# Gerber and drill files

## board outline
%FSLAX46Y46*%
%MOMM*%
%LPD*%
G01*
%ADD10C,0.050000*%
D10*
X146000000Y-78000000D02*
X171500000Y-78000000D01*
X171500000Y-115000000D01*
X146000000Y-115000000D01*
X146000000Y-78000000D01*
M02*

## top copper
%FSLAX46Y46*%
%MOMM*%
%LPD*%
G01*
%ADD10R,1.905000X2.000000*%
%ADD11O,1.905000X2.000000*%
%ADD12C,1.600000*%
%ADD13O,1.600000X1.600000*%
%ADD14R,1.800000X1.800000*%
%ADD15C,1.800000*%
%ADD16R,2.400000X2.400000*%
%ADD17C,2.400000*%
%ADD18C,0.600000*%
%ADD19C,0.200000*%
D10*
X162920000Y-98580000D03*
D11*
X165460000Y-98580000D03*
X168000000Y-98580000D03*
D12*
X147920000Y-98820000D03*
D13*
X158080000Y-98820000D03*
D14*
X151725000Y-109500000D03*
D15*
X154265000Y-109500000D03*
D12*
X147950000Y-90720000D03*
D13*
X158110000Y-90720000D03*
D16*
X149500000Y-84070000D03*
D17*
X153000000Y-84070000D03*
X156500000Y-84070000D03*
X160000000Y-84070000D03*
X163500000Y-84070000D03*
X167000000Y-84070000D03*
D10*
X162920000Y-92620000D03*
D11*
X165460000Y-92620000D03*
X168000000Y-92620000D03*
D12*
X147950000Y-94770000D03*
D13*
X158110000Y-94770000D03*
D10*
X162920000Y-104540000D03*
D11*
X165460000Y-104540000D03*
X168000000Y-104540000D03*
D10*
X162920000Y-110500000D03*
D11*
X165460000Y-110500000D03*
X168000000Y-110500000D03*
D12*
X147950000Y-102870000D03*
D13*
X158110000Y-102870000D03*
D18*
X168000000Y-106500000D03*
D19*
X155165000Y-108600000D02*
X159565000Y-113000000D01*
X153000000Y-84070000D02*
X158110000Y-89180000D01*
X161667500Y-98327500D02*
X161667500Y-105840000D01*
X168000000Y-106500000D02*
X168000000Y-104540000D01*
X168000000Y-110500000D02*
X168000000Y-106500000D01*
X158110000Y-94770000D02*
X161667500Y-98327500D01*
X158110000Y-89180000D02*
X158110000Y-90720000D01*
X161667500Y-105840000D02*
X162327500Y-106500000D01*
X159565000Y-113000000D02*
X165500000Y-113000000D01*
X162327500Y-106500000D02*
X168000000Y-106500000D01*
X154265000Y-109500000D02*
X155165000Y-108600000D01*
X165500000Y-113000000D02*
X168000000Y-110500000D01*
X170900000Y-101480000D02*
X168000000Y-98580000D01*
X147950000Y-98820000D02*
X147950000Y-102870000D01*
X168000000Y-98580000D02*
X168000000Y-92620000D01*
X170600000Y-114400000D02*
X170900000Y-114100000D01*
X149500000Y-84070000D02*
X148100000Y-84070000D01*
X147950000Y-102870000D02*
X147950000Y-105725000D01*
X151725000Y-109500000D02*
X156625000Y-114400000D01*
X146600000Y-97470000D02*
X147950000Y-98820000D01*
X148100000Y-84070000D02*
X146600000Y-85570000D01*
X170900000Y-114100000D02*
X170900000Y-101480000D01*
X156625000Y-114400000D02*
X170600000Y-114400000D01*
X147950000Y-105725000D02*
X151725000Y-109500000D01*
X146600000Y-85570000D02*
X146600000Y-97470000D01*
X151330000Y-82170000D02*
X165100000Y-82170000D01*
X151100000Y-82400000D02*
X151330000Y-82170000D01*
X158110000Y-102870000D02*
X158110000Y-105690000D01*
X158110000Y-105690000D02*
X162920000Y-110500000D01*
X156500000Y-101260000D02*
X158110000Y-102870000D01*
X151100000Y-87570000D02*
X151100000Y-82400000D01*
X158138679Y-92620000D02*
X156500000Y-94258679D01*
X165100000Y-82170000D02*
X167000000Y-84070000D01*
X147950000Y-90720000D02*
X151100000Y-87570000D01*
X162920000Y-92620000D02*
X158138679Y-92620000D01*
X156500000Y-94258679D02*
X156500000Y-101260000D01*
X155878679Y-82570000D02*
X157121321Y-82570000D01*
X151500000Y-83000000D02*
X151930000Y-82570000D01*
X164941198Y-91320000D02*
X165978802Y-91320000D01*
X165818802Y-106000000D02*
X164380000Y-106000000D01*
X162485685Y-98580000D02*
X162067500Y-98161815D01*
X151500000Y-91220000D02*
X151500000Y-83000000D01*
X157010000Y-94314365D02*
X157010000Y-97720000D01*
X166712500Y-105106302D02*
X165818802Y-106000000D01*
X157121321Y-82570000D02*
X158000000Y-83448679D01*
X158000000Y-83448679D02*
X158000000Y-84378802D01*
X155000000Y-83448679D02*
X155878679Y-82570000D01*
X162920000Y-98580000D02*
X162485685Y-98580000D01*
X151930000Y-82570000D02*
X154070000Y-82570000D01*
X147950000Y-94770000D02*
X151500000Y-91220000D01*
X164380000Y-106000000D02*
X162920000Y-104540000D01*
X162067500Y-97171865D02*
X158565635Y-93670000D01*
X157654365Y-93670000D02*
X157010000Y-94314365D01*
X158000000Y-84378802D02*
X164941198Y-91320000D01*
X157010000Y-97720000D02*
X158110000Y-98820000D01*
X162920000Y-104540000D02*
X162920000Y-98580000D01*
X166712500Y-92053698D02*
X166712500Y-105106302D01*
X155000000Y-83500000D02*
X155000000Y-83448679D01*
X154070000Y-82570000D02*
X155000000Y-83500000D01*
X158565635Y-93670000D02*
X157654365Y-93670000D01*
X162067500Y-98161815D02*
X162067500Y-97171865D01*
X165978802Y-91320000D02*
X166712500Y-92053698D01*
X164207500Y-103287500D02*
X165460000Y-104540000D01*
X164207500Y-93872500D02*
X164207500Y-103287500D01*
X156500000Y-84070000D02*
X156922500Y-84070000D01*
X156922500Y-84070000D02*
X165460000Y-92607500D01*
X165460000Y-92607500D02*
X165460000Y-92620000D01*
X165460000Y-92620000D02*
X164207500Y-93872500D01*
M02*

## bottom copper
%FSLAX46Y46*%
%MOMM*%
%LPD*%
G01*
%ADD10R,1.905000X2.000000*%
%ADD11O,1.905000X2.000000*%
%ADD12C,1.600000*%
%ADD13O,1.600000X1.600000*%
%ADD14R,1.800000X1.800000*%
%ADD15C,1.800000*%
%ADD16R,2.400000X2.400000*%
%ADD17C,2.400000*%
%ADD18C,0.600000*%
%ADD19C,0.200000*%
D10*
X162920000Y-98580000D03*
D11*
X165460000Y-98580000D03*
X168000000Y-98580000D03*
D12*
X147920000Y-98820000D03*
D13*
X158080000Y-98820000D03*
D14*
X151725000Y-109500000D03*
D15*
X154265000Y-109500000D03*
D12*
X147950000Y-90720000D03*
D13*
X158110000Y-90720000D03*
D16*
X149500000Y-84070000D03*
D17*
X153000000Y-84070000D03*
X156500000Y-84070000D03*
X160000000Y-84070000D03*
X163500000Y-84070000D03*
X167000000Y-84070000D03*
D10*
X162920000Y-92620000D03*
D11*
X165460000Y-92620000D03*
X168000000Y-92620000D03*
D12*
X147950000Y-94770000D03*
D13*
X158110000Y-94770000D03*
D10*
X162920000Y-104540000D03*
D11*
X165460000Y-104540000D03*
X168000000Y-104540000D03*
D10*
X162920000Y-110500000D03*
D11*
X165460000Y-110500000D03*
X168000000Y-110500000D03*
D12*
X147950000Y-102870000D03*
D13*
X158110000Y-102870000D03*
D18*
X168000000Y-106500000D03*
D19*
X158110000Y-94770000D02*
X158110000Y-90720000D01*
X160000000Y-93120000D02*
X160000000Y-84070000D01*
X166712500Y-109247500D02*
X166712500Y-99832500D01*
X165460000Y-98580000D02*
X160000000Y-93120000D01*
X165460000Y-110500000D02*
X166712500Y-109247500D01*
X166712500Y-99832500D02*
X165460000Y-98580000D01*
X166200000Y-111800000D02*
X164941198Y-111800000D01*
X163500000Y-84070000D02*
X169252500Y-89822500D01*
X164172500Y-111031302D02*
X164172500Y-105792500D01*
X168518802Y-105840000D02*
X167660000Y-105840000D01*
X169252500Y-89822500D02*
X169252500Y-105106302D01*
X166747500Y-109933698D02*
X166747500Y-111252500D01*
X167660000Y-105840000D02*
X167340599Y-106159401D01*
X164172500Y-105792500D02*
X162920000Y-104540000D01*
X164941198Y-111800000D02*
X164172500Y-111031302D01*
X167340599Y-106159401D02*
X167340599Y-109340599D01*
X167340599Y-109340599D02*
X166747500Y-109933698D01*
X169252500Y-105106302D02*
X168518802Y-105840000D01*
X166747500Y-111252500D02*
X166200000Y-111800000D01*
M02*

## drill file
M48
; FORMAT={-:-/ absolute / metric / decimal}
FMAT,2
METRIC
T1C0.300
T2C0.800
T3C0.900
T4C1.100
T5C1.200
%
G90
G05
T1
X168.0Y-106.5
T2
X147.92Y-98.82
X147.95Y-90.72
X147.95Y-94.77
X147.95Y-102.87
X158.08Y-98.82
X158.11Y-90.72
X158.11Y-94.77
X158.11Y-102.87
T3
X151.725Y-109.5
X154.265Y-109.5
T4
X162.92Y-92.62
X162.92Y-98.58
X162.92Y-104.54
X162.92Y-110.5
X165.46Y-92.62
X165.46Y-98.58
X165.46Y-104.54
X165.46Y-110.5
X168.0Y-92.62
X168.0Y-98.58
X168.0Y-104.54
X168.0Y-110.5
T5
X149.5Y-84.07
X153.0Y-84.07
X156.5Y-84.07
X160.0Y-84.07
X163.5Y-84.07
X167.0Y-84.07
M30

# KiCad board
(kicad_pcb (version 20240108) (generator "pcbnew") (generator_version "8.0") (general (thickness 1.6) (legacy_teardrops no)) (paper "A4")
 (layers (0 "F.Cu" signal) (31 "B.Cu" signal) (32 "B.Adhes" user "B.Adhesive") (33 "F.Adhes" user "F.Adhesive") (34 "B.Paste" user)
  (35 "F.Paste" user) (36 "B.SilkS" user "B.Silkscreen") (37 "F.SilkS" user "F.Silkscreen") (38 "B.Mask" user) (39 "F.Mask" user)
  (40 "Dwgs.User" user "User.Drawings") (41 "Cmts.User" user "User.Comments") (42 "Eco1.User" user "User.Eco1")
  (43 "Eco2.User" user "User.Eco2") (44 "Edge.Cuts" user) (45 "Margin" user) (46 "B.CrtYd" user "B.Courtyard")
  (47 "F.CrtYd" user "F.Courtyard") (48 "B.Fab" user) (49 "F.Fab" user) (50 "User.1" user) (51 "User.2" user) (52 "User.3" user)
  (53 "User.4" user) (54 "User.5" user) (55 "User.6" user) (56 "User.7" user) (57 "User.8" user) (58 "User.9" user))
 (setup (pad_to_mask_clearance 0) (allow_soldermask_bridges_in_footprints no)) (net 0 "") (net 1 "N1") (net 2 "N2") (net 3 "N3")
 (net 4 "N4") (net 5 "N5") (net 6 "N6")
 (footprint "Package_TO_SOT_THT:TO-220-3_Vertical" (layer "F.Cu") (at 162.92 98.58)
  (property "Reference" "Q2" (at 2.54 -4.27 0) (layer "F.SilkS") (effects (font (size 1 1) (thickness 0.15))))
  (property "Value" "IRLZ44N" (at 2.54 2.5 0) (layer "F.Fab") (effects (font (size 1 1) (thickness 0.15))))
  (pad "1" thru_hole rect (at 0 0) (size 1.905 2) (drill 1.1) (layers "*.Cu" "*.Mask") (remove_unused_layers no) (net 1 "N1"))
  (pad "2" thru_hole oval (at 2.54 0) (size 1.905 2) (drill 1.1) (layers "*.Cu" "*.Mask") (remove_unused_layers no) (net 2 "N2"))
  (pad "3" thru_hole oval (at 5.08 0) (size 1.905 2) (drill 1.1) (layers "*.Cu" "*.Mask") (remove_unused_layers no) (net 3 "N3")))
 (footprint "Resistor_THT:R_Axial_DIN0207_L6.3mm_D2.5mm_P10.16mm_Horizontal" (layer "F.Cu") (at 147.92 98.82)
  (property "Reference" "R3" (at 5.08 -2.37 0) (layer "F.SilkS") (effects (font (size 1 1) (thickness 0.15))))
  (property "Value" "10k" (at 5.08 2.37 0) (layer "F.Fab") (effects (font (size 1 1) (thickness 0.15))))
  (pad "1" thru_hole circle (at 0 0) (size 1.6 1.6) (drill 0.8) (layers "*.Cu" "*.Mask") (remove_unused_layers no) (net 3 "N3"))
  (pad "2" thru_hole oval (at 10.16 0) (size 1.6 1.6) (drill 0.8) (layers "*.Cu" "*.Mask") (remove_unused_layers no) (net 1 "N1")))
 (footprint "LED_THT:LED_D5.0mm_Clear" (layer "F.Cu") (at 151.725 109.5)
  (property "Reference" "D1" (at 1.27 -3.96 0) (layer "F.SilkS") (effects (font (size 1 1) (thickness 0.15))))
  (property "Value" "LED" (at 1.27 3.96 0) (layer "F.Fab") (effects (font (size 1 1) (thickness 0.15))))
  (pad "1" thru_hole rect (at 0 0) (size 1.8 1.8) (drill 0.9) (layers "*.Cu" "*.Mask") (remove_unused_layers no) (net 3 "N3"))
  (pad "2" thru_hole circle (at 2.54 0) (size 1.8 1.8) (drill 0.9) (layers "*.Cu" "*.Mask") (remove_unused_layers no) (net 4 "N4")))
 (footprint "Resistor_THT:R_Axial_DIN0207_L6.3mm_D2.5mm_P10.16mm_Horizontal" (layer "F.Cu") (at 147.95 90.72)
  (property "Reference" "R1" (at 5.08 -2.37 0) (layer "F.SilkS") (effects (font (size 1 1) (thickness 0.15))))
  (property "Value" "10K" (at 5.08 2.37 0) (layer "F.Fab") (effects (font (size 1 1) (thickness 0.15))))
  (pad "1" thru_hole circle (at 0 0) (size 1.6 1.6) (drill 0.8) (layers "*.Cu" "*.Mask") (remove_unused_layers no) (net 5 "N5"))
  (pad "2" thru_hole oval (at 10.16 0) (size 1.6 1.6) (drill 0.8) (layers "*.Cu" "*.Mask") (remove_unused_layers no) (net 4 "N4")))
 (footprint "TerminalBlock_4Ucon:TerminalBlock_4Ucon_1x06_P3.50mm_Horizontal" (layer "F.Cu") (at 149.5 84.07)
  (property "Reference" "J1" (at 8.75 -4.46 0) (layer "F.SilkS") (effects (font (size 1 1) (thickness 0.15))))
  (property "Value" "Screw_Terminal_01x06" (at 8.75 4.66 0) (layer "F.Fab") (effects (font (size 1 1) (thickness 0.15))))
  (pad "1" thru_hole rect (at 0 0) (size 2.4 2.4) (drill 1.2) (layers "*.Cu" "*.Mask") (remove_unused_layers no) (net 3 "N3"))
  (pad "2" thru_hole circle (at 3.5 0) (size 2.4 2.4) (drill 1.2) (layers "*.Cu" "*.Mask") (remove_unused_layers no) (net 4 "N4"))
  (pad "3" thru_hole circle (at 7 0) (size 2.4 2.4) (drill 1.2) (layers "*.Cu" "*.Mask") (remove_unused_layers no) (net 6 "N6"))
  (pad "4" thru_hole circle (at 10.5 0) (size 2.4 2.4) (drill 1.2) (layers "*.Cu" "*.Mask") (remove_unused_layers no) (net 2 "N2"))
  (pad "5" thru_hole circle (at 14 0) (size 2.4 2.4) (drill 1.2) (layers "*.Cu" "*.Mask") (remove_unused_layers no) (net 1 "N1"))
  (pad "6" thru_hole circle (at 17.5 0) (size 2.4 2.4) (drill 1.2) (layers "*.Cu" "*.Mask") (remove_unused_layers no) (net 5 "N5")))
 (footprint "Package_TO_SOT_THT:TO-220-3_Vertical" (layer "F.Cu") (at 162.92 92.62)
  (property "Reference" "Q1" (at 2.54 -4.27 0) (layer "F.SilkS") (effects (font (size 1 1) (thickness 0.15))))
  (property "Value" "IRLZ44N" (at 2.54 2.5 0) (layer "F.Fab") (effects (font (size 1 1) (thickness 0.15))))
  (pad "1" thru_hole rect (at 0 0) (size 1.905 2) (drill 1.1) (layers "*.Cu" "*.Mask") (remove_unused_layers no) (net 5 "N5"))
  (pad "2" thru_hole oval (at 2.54 0) (size 1.905 2) (drill 1.1) (layers "*.Cu" "*.Mask") (remove_unused_layers no) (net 6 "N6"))
  (pad "3" thru_hole oval (at 5.08 0) (size 1.905 2) (drill 1.1) (layers "*.Cu" "*.Mask") (remove_unused_layers no) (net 3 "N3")))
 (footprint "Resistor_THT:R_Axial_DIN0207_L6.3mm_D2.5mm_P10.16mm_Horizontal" (layer "F.Cu") (at 147.95 94.77)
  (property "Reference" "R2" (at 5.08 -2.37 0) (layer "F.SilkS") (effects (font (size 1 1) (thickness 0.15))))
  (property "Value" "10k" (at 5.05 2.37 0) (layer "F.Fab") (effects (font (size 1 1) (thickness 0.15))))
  (pad "1" thru_hole circle (at 0 0) (size 1.6 1.6) (drill 0.8) (layers "*.Cu" "*.Mask") (remove_unused_layers no) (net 1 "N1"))
  (pad "2" thru_hole oval (at 10.16 0) (size 1.6 1.6) (drill 0.8) (layers "*.Cu" "*.Mask") (remove_unused_layers no) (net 4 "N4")))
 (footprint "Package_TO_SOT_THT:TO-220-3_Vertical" (layer "F.Cu") (at 162.92 104.54)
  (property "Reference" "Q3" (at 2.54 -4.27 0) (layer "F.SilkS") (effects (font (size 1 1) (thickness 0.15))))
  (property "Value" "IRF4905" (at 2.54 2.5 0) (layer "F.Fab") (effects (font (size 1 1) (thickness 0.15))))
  (pad "1" thru_hole rect (at 0 0) (size 1.905 2) (drill 1.1) (layers "*.Cu" "*.Mask") (remove_unused_layers no) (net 1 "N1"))
  (pad "2" thru_hole oval (at 2.54 0) (size 1.905 2) (drill 1.1) (layers "*.Cu" "*.Mask") (remove_unused_layers no) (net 6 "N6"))
  (pad "3" thru_hole oval (at 5.08 0) (size 1.905 2) (drill 1.1) (layers "*.Cu" "*.Mask") (remove_unused_layers no) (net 4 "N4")))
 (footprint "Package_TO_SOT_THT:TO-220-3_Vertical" (layer "F.Cu") (at 162.92 110.5)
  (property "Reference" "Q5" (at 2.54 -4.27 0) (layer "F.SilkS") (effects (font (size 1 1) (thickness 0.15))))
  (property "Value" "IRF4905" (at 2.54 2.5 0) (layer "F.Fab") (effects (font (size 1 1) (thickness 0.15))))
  (pad "1" thru_hole rect (at 0 0) (size 1.905 2) (drill 1.1) (layers "*.Cu" "*.Mask") (remove_unused_layers no) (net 5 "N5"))
  (pad "2" thru_hole oval (at 2.54 0) (size 1.905 2) (drill 1.1) (layers "*.Cu" "*.Mask") (remove_unused_layers no) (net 2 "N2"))
  (pad "3" thru_hole oval (at 5.08 0) (size 1.905 2) (drill 1.1) (layers "*.Cu" "*.Mask") (remove_unused_layers no) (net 4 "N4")))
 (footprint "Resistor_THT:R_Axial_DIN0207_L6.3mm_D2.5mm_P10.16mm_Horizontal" (layer "F.Cu") (at 147.95 102.87)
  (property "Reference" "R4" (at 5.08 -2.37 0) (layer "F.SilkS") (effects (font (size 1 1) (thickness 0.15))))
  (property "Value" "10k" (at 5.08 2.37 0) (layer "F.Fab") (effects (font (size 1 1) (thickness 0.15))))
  (pad "1" thru_hole circle (at 0 0) (size 1.6 1.6) (drill 0.8) (layers "*.Cu" "*.Mask") (remove_unused_layers no) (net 3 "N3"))
  (pad "2" thru_hole oval (at 10.16 0) (size 1.6 1.6) (drill 0.8) (layers "*.Cu" "*.Mask") (remove_unused_layers no) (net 5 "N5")))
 (gr_rect (start 146 78) (end 171.5 115) (stroke (width 0.05) (type default)) (fill none) (layer "Edge.Cuts"))
 (segment (start 155.165 108.6) (end 159.565 113) (width 0.2) (layer "F.Cu") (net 4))
 (segment (start 153 84.07) (end 158.11 89.18) (width 0.2) (layer "F.Cu") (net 4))
 (segment (start 161.6675 98.3275) (end 161.6675 105.84) (width 0.2) (layer "F.Cu") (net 4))
 (segment (start 168 106.5) (end 168 104.54) (width 0.2) (layer "F.Cu") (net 4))
 (segment (start 168 110.5) (end 168 106.5) (width 0.2) (layer "F.Cu") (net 4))
 (segment (start 158.11 94.77) (end 161.6675 98.3275) (width 0.2) (layer "F.Cu") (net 4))
 (segment (start 158.11 89.18) (end 158.11 90.72) (width 0.2) (layer "F.Cu") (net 4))
 (segment (start 161.6675 105.84) (end 162.3275 106.5) (width 0.2) (layer "F.Cu") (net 4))
 (segment (start 159.565 113) (end 165.5 113) (width 0.2) (layer "F.Cu") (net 4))
 (segment (start 162.3275 106.5) (end 168 106.5) (width 0.2) (layer "F.Cu") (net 4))
 (segment (start 154.265 109.5) (end 155.165 108.6) (width 0.2) (layer "F.Cu") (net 4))
 (segment (start 165.5 113) (end 168 110.5) (width 0.2) (layer "F.Cu") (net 4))
 (via (at 168 106.5) (size 0.6) (drill 0.3) (layers "F.Cu" "B.Cu") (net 4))
 (segment (start 158.11 94.77) (end 158.11 90.72) (width 0.2) (layer "B.Cu") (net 4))
 (segment (start 170.9 101.48) (end 168 98.58) (width 0.2) (layer "F.Cu") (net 3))
 (segment (start 147.95 98.82) (end 147.95 102.87) (width 0.2) (layer "F.Cu") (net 3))
 (segment (start 168 98.58) (end 168 92.62) (width 0.2) (layer "F.Cu") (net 3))
 (segment (start 170.6 114.4) (end 170.9 114.1) (width 0.2) (layer "F.Cu") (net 3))
 (segment (start 149.5 84.07) (end 148.1 84.07) (width 0.2) (layer "F.Cu") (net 3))
 (segment (start 147.95 102.87) (end 147.95 105.725) (width 0.2) (layer "F.Cu") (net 3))
 (segment (start 151.725 109.5) (end 156.625 114.4) (width 0.2) (layer "F.Cu") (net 3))
 (segment (start 146.6 97.47) (end 147.95 98.82) (width 0.2) (layer "F.Cu") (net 3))
 (segment (start 148.1 84.07) (end 146.6 85.57) (width 0.2) (layer "F.Cu") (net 3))
 (segment (start 170.9 114.1) (end 170.9 101.48) (width 0.2) (layer "F.Cu") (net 3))
 (segment (start 156.625 114.4) (end 170.6 114.4) (width 0.2) (layer "F.Cu") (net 3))
 (segment (start 147.95 105.725) (end 151.725 109.5) (width 0.2) (layer "F.Cu") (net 3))
 (segment (start 146.6 85.57) (end 146.6 97.47) (width 0.2) (layer "F.Cu") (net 3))
 (segment (start 160 93.12) (end 160 84.07) (width 0.2) (layer "B.Cu") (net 2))
 (segment (start 166.7125 109.2475) (end 166.7125 99.8325) (width 0.2) (layer "B.Cu") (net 2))
 (segment (start 165.46 98.58) (end 160 93.12) (width 0.2) (layer "B.Cu") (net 2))
 (segment (start 165.46 110.5) (end 166.7125 109.2475) (width 0.2) (layer "B.Cu") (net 2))
 (segment (start 166.7125 99.8325) (end 165.46 98.58) (width 0.2) (layer "B.Cu") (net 2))
 (segment (start 151.33 82.17) (end 165.1 82.17) (width 0.2) (layer "F.Cu") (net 5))
 (segment (start 151.1 82.4) (end 151.33 82.17) (width 0.2) (layer "F.Cu") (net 5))
 (segment (start 158.11 102.87) (end 158.11 105.69) (width 0.2) (layer "F.Cu") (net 5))
 (segment (start 158.11 105.69) (end 162.92 110.5) (width 0.2) (layer "F.Cu") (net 5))
 (segment (start 156.5 101.26) (end 158.11 102.87) (width 0.2) (layer "F.Cu") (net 5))
 (segment (start 151.1 87.57) (end 151.1 82.4) (width 0.2) (layer "F.Cu") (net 5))
 (segment (start 158.138679 92.62) (end 156.5 94.258679) (width 0.2) (layer "F.Cu") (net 5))
 (segment (start 165.1 82.17) (end 167 84.07) (width 0.2) (layer "F.Cu") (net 5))
 (segment (start 147.95 90.72) (end 151.1 87.57) (width 0.2) (layer "F.Cu") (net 5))
 (segment (start 162.92 92.62) (end 158.138679 92.62) (width 0.2) (layer "F.Cu") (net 5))
 (segment (start 156.5 94.258679) (end 156.5 101.26) (width 0.2) (layer "F.Cu") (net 5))
 (segment (start 155.878679 82.57) (end 157.121321 82.57) (width 0.2) (layer "F.Cu") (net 1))
 (segment (start 151.5 83) (end 151.93 82.57) (width 0.2) (layer "F.Cu") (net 1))
 (segment (start 164.941198 91.32) (end 165.978802 91.32) (width 0.2) (layer "F.Cu") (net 1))
 (segment (start 165.818802 106) (end 164.38 106) (width 0.2) (layer "F.Cu") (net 1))
 (segment (start 162.485685 98.58) (end 162.0675 98.161815) (width 0.2) (layer "F.Cu") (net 1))
 (segment (start 151.5 91.22) (end 151.5 83) (width 0.2) (layer "F.Cu") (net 1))
 (segment (start 157.01 94.314365) (end 157.01 97.72) (width 0.2) (layer "F.Cu") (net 1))
 (segment (start 166.7125 105.106302) (end 165.818802 106) (width 0.2) (layer "F.Cu") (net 1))
 (segment (start 157.121321 82.57) (end 158 83.448679) (width 0.2) (layer "F.Cu") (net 1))
 (segment (start 158 83.448679) (end 158 84.378802) (width 0.2) (layer "F.Cu") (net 1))
 (segment (start 155 83.448679) (end 155.878679 82.57) (width 0.2) (layer "F.Cu") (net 1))
 (segment (start 162.92 98.58) (end 162.485685 98.58) (width 0.2) (layer "F.Cu") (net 1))
 (segment (start 151.93 82.57) (end 154.07 82.57) (width 0.2) (layer "F.Cu") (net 1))
 (segment (start 147.95 94.77) (end 151.5 91.22) (width 0.2) (layer "F.Cu") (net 1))
 (segment (start 164.38 106) (end 162.92 104.54) (width 0.2) (layer "F.Cu") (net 1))
 (segment (start 162.0675 97.171865) (end 158.565635 93.67) (width 0.2) (layer "F.Cu") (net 1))
 (segment (start 157.654365 93.67) (end 157.01 94.314365) (width 0.2) (layer "F.Cu") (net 1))
 (segment (start 158 84.378802) (end 164.941198 91.32) (width 0.2) (layer "F.Cu") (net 1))
 (segment (start 157.01 97.72) (end 158.11 98.82) (width 0.2) (layer "F.Cu") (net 1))
 (segment (start 162.92 104.54) (end 162.92 98.58) (width 0.2) (layer "F.Cu") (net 1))
 (segment (start 166.7125 92.053698) (end 166.7125 105.106302) (width 0.2) (layer "F.Cu") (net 1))
 (segment (start 155 83.5) (end 155 83.448679) (width 0.2) (layer "F.Cu") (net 1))
 (segment (start 154.07 82.57) (end 155 83.5) (width 0.2) (layer "F.Cu") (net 1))
 (segment (start 158.565635 93.67) (end 157.654365 93.67) (width 0.2) (layer "F.Cu") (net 1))
 (segment (start 162.0675 98.161815) (end 162.0675 97.171865) (width 0.2) (layer "F.Cu") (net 1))
 (segment (start 165.978802 91.32) (end 166.7125 92.053698) (width 0.2) (layer "F.Cu") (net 1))
 (segment (start 166.2 111.8) (end 164.941198 111.8) (width 0.2) (layer "B.Cu") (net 1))
 (segment (start 163.5 84.07) (end 169.2525 89.8225) (width 0.2) (layer "B.Cu") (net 1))
 (segment (start 164.1725 111.031302) (end 164.1725 105.7925) (width 0.2) (layer "B.Cu") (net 1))
 (segment (start 168.518802 105.84) (end 167.66 105.84) (width 0.2) (layer "B.Cu") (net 1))
 (segment (start 169.2525 89.8225) (end 169.2525 105.106302) (width 0.2) (layer "B.Cu") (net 1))
 (segment (start 166.7475 109.933698) (end 166.7475 111.2525) (width 0.2) (layer "B.Cu") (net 1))
 (segment (start 167.66 105.84) (end 167.340599 106.159401) (width 0.2) (layer "B.Cu") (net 1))
 (segment (start 164.1725 105.7925) (end 162.92 104.54) (width 0.2) (layer "B.Cu") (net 1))
 (segment (start 164.941198 111.8) (end 164.1725 111.031302) (width 0.2) (layer "B.Cu") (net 1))
 (segment (start 167.340599 106.159401) (end 167.340599 109.340599) (width 0.2) (layer "B.Cu") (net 1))
 (segment (start 167.340599 109.340599) (end 166.7475 109.933698) (width 0.2) (layer "B.Cu") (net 1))
 (segment (start 169.2525 105.106302) (end 168.518802 105.84) (width 0.2) (layer "B.Cu") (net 1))
 (segment (start 166.7475 111.2525) (end 166.2 111.8) (width 0.2) (layer "B.Cu") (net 1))
 (segment (start 164.2075 103.2875) (end 165.46 104.54) (width 0.2) (layer "F.Cu") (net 6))
 (segment (start 164.2075 93.8725) (end 164.2075 103.2875) (width 0.2) (layer "F.Cu") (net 6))
 (segment (start 156.5 84.07) (end 156.9225 84.07) (width 0.2) (layer "F.Cu") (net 6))
 (segment (start 156.9225 84.07) (end 165.46 92.6075) (width 0.2) (layer "F.Cu") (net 6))
 (segment (start 165.46 92.6075) (end 165.46 92.62) (width 0.2) (layer "F.Cu") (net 6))
 (segment (start 165.46 92.62) (end 164.2075 93.8725) (width 0.2) (layer "F.Cu") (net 6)))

